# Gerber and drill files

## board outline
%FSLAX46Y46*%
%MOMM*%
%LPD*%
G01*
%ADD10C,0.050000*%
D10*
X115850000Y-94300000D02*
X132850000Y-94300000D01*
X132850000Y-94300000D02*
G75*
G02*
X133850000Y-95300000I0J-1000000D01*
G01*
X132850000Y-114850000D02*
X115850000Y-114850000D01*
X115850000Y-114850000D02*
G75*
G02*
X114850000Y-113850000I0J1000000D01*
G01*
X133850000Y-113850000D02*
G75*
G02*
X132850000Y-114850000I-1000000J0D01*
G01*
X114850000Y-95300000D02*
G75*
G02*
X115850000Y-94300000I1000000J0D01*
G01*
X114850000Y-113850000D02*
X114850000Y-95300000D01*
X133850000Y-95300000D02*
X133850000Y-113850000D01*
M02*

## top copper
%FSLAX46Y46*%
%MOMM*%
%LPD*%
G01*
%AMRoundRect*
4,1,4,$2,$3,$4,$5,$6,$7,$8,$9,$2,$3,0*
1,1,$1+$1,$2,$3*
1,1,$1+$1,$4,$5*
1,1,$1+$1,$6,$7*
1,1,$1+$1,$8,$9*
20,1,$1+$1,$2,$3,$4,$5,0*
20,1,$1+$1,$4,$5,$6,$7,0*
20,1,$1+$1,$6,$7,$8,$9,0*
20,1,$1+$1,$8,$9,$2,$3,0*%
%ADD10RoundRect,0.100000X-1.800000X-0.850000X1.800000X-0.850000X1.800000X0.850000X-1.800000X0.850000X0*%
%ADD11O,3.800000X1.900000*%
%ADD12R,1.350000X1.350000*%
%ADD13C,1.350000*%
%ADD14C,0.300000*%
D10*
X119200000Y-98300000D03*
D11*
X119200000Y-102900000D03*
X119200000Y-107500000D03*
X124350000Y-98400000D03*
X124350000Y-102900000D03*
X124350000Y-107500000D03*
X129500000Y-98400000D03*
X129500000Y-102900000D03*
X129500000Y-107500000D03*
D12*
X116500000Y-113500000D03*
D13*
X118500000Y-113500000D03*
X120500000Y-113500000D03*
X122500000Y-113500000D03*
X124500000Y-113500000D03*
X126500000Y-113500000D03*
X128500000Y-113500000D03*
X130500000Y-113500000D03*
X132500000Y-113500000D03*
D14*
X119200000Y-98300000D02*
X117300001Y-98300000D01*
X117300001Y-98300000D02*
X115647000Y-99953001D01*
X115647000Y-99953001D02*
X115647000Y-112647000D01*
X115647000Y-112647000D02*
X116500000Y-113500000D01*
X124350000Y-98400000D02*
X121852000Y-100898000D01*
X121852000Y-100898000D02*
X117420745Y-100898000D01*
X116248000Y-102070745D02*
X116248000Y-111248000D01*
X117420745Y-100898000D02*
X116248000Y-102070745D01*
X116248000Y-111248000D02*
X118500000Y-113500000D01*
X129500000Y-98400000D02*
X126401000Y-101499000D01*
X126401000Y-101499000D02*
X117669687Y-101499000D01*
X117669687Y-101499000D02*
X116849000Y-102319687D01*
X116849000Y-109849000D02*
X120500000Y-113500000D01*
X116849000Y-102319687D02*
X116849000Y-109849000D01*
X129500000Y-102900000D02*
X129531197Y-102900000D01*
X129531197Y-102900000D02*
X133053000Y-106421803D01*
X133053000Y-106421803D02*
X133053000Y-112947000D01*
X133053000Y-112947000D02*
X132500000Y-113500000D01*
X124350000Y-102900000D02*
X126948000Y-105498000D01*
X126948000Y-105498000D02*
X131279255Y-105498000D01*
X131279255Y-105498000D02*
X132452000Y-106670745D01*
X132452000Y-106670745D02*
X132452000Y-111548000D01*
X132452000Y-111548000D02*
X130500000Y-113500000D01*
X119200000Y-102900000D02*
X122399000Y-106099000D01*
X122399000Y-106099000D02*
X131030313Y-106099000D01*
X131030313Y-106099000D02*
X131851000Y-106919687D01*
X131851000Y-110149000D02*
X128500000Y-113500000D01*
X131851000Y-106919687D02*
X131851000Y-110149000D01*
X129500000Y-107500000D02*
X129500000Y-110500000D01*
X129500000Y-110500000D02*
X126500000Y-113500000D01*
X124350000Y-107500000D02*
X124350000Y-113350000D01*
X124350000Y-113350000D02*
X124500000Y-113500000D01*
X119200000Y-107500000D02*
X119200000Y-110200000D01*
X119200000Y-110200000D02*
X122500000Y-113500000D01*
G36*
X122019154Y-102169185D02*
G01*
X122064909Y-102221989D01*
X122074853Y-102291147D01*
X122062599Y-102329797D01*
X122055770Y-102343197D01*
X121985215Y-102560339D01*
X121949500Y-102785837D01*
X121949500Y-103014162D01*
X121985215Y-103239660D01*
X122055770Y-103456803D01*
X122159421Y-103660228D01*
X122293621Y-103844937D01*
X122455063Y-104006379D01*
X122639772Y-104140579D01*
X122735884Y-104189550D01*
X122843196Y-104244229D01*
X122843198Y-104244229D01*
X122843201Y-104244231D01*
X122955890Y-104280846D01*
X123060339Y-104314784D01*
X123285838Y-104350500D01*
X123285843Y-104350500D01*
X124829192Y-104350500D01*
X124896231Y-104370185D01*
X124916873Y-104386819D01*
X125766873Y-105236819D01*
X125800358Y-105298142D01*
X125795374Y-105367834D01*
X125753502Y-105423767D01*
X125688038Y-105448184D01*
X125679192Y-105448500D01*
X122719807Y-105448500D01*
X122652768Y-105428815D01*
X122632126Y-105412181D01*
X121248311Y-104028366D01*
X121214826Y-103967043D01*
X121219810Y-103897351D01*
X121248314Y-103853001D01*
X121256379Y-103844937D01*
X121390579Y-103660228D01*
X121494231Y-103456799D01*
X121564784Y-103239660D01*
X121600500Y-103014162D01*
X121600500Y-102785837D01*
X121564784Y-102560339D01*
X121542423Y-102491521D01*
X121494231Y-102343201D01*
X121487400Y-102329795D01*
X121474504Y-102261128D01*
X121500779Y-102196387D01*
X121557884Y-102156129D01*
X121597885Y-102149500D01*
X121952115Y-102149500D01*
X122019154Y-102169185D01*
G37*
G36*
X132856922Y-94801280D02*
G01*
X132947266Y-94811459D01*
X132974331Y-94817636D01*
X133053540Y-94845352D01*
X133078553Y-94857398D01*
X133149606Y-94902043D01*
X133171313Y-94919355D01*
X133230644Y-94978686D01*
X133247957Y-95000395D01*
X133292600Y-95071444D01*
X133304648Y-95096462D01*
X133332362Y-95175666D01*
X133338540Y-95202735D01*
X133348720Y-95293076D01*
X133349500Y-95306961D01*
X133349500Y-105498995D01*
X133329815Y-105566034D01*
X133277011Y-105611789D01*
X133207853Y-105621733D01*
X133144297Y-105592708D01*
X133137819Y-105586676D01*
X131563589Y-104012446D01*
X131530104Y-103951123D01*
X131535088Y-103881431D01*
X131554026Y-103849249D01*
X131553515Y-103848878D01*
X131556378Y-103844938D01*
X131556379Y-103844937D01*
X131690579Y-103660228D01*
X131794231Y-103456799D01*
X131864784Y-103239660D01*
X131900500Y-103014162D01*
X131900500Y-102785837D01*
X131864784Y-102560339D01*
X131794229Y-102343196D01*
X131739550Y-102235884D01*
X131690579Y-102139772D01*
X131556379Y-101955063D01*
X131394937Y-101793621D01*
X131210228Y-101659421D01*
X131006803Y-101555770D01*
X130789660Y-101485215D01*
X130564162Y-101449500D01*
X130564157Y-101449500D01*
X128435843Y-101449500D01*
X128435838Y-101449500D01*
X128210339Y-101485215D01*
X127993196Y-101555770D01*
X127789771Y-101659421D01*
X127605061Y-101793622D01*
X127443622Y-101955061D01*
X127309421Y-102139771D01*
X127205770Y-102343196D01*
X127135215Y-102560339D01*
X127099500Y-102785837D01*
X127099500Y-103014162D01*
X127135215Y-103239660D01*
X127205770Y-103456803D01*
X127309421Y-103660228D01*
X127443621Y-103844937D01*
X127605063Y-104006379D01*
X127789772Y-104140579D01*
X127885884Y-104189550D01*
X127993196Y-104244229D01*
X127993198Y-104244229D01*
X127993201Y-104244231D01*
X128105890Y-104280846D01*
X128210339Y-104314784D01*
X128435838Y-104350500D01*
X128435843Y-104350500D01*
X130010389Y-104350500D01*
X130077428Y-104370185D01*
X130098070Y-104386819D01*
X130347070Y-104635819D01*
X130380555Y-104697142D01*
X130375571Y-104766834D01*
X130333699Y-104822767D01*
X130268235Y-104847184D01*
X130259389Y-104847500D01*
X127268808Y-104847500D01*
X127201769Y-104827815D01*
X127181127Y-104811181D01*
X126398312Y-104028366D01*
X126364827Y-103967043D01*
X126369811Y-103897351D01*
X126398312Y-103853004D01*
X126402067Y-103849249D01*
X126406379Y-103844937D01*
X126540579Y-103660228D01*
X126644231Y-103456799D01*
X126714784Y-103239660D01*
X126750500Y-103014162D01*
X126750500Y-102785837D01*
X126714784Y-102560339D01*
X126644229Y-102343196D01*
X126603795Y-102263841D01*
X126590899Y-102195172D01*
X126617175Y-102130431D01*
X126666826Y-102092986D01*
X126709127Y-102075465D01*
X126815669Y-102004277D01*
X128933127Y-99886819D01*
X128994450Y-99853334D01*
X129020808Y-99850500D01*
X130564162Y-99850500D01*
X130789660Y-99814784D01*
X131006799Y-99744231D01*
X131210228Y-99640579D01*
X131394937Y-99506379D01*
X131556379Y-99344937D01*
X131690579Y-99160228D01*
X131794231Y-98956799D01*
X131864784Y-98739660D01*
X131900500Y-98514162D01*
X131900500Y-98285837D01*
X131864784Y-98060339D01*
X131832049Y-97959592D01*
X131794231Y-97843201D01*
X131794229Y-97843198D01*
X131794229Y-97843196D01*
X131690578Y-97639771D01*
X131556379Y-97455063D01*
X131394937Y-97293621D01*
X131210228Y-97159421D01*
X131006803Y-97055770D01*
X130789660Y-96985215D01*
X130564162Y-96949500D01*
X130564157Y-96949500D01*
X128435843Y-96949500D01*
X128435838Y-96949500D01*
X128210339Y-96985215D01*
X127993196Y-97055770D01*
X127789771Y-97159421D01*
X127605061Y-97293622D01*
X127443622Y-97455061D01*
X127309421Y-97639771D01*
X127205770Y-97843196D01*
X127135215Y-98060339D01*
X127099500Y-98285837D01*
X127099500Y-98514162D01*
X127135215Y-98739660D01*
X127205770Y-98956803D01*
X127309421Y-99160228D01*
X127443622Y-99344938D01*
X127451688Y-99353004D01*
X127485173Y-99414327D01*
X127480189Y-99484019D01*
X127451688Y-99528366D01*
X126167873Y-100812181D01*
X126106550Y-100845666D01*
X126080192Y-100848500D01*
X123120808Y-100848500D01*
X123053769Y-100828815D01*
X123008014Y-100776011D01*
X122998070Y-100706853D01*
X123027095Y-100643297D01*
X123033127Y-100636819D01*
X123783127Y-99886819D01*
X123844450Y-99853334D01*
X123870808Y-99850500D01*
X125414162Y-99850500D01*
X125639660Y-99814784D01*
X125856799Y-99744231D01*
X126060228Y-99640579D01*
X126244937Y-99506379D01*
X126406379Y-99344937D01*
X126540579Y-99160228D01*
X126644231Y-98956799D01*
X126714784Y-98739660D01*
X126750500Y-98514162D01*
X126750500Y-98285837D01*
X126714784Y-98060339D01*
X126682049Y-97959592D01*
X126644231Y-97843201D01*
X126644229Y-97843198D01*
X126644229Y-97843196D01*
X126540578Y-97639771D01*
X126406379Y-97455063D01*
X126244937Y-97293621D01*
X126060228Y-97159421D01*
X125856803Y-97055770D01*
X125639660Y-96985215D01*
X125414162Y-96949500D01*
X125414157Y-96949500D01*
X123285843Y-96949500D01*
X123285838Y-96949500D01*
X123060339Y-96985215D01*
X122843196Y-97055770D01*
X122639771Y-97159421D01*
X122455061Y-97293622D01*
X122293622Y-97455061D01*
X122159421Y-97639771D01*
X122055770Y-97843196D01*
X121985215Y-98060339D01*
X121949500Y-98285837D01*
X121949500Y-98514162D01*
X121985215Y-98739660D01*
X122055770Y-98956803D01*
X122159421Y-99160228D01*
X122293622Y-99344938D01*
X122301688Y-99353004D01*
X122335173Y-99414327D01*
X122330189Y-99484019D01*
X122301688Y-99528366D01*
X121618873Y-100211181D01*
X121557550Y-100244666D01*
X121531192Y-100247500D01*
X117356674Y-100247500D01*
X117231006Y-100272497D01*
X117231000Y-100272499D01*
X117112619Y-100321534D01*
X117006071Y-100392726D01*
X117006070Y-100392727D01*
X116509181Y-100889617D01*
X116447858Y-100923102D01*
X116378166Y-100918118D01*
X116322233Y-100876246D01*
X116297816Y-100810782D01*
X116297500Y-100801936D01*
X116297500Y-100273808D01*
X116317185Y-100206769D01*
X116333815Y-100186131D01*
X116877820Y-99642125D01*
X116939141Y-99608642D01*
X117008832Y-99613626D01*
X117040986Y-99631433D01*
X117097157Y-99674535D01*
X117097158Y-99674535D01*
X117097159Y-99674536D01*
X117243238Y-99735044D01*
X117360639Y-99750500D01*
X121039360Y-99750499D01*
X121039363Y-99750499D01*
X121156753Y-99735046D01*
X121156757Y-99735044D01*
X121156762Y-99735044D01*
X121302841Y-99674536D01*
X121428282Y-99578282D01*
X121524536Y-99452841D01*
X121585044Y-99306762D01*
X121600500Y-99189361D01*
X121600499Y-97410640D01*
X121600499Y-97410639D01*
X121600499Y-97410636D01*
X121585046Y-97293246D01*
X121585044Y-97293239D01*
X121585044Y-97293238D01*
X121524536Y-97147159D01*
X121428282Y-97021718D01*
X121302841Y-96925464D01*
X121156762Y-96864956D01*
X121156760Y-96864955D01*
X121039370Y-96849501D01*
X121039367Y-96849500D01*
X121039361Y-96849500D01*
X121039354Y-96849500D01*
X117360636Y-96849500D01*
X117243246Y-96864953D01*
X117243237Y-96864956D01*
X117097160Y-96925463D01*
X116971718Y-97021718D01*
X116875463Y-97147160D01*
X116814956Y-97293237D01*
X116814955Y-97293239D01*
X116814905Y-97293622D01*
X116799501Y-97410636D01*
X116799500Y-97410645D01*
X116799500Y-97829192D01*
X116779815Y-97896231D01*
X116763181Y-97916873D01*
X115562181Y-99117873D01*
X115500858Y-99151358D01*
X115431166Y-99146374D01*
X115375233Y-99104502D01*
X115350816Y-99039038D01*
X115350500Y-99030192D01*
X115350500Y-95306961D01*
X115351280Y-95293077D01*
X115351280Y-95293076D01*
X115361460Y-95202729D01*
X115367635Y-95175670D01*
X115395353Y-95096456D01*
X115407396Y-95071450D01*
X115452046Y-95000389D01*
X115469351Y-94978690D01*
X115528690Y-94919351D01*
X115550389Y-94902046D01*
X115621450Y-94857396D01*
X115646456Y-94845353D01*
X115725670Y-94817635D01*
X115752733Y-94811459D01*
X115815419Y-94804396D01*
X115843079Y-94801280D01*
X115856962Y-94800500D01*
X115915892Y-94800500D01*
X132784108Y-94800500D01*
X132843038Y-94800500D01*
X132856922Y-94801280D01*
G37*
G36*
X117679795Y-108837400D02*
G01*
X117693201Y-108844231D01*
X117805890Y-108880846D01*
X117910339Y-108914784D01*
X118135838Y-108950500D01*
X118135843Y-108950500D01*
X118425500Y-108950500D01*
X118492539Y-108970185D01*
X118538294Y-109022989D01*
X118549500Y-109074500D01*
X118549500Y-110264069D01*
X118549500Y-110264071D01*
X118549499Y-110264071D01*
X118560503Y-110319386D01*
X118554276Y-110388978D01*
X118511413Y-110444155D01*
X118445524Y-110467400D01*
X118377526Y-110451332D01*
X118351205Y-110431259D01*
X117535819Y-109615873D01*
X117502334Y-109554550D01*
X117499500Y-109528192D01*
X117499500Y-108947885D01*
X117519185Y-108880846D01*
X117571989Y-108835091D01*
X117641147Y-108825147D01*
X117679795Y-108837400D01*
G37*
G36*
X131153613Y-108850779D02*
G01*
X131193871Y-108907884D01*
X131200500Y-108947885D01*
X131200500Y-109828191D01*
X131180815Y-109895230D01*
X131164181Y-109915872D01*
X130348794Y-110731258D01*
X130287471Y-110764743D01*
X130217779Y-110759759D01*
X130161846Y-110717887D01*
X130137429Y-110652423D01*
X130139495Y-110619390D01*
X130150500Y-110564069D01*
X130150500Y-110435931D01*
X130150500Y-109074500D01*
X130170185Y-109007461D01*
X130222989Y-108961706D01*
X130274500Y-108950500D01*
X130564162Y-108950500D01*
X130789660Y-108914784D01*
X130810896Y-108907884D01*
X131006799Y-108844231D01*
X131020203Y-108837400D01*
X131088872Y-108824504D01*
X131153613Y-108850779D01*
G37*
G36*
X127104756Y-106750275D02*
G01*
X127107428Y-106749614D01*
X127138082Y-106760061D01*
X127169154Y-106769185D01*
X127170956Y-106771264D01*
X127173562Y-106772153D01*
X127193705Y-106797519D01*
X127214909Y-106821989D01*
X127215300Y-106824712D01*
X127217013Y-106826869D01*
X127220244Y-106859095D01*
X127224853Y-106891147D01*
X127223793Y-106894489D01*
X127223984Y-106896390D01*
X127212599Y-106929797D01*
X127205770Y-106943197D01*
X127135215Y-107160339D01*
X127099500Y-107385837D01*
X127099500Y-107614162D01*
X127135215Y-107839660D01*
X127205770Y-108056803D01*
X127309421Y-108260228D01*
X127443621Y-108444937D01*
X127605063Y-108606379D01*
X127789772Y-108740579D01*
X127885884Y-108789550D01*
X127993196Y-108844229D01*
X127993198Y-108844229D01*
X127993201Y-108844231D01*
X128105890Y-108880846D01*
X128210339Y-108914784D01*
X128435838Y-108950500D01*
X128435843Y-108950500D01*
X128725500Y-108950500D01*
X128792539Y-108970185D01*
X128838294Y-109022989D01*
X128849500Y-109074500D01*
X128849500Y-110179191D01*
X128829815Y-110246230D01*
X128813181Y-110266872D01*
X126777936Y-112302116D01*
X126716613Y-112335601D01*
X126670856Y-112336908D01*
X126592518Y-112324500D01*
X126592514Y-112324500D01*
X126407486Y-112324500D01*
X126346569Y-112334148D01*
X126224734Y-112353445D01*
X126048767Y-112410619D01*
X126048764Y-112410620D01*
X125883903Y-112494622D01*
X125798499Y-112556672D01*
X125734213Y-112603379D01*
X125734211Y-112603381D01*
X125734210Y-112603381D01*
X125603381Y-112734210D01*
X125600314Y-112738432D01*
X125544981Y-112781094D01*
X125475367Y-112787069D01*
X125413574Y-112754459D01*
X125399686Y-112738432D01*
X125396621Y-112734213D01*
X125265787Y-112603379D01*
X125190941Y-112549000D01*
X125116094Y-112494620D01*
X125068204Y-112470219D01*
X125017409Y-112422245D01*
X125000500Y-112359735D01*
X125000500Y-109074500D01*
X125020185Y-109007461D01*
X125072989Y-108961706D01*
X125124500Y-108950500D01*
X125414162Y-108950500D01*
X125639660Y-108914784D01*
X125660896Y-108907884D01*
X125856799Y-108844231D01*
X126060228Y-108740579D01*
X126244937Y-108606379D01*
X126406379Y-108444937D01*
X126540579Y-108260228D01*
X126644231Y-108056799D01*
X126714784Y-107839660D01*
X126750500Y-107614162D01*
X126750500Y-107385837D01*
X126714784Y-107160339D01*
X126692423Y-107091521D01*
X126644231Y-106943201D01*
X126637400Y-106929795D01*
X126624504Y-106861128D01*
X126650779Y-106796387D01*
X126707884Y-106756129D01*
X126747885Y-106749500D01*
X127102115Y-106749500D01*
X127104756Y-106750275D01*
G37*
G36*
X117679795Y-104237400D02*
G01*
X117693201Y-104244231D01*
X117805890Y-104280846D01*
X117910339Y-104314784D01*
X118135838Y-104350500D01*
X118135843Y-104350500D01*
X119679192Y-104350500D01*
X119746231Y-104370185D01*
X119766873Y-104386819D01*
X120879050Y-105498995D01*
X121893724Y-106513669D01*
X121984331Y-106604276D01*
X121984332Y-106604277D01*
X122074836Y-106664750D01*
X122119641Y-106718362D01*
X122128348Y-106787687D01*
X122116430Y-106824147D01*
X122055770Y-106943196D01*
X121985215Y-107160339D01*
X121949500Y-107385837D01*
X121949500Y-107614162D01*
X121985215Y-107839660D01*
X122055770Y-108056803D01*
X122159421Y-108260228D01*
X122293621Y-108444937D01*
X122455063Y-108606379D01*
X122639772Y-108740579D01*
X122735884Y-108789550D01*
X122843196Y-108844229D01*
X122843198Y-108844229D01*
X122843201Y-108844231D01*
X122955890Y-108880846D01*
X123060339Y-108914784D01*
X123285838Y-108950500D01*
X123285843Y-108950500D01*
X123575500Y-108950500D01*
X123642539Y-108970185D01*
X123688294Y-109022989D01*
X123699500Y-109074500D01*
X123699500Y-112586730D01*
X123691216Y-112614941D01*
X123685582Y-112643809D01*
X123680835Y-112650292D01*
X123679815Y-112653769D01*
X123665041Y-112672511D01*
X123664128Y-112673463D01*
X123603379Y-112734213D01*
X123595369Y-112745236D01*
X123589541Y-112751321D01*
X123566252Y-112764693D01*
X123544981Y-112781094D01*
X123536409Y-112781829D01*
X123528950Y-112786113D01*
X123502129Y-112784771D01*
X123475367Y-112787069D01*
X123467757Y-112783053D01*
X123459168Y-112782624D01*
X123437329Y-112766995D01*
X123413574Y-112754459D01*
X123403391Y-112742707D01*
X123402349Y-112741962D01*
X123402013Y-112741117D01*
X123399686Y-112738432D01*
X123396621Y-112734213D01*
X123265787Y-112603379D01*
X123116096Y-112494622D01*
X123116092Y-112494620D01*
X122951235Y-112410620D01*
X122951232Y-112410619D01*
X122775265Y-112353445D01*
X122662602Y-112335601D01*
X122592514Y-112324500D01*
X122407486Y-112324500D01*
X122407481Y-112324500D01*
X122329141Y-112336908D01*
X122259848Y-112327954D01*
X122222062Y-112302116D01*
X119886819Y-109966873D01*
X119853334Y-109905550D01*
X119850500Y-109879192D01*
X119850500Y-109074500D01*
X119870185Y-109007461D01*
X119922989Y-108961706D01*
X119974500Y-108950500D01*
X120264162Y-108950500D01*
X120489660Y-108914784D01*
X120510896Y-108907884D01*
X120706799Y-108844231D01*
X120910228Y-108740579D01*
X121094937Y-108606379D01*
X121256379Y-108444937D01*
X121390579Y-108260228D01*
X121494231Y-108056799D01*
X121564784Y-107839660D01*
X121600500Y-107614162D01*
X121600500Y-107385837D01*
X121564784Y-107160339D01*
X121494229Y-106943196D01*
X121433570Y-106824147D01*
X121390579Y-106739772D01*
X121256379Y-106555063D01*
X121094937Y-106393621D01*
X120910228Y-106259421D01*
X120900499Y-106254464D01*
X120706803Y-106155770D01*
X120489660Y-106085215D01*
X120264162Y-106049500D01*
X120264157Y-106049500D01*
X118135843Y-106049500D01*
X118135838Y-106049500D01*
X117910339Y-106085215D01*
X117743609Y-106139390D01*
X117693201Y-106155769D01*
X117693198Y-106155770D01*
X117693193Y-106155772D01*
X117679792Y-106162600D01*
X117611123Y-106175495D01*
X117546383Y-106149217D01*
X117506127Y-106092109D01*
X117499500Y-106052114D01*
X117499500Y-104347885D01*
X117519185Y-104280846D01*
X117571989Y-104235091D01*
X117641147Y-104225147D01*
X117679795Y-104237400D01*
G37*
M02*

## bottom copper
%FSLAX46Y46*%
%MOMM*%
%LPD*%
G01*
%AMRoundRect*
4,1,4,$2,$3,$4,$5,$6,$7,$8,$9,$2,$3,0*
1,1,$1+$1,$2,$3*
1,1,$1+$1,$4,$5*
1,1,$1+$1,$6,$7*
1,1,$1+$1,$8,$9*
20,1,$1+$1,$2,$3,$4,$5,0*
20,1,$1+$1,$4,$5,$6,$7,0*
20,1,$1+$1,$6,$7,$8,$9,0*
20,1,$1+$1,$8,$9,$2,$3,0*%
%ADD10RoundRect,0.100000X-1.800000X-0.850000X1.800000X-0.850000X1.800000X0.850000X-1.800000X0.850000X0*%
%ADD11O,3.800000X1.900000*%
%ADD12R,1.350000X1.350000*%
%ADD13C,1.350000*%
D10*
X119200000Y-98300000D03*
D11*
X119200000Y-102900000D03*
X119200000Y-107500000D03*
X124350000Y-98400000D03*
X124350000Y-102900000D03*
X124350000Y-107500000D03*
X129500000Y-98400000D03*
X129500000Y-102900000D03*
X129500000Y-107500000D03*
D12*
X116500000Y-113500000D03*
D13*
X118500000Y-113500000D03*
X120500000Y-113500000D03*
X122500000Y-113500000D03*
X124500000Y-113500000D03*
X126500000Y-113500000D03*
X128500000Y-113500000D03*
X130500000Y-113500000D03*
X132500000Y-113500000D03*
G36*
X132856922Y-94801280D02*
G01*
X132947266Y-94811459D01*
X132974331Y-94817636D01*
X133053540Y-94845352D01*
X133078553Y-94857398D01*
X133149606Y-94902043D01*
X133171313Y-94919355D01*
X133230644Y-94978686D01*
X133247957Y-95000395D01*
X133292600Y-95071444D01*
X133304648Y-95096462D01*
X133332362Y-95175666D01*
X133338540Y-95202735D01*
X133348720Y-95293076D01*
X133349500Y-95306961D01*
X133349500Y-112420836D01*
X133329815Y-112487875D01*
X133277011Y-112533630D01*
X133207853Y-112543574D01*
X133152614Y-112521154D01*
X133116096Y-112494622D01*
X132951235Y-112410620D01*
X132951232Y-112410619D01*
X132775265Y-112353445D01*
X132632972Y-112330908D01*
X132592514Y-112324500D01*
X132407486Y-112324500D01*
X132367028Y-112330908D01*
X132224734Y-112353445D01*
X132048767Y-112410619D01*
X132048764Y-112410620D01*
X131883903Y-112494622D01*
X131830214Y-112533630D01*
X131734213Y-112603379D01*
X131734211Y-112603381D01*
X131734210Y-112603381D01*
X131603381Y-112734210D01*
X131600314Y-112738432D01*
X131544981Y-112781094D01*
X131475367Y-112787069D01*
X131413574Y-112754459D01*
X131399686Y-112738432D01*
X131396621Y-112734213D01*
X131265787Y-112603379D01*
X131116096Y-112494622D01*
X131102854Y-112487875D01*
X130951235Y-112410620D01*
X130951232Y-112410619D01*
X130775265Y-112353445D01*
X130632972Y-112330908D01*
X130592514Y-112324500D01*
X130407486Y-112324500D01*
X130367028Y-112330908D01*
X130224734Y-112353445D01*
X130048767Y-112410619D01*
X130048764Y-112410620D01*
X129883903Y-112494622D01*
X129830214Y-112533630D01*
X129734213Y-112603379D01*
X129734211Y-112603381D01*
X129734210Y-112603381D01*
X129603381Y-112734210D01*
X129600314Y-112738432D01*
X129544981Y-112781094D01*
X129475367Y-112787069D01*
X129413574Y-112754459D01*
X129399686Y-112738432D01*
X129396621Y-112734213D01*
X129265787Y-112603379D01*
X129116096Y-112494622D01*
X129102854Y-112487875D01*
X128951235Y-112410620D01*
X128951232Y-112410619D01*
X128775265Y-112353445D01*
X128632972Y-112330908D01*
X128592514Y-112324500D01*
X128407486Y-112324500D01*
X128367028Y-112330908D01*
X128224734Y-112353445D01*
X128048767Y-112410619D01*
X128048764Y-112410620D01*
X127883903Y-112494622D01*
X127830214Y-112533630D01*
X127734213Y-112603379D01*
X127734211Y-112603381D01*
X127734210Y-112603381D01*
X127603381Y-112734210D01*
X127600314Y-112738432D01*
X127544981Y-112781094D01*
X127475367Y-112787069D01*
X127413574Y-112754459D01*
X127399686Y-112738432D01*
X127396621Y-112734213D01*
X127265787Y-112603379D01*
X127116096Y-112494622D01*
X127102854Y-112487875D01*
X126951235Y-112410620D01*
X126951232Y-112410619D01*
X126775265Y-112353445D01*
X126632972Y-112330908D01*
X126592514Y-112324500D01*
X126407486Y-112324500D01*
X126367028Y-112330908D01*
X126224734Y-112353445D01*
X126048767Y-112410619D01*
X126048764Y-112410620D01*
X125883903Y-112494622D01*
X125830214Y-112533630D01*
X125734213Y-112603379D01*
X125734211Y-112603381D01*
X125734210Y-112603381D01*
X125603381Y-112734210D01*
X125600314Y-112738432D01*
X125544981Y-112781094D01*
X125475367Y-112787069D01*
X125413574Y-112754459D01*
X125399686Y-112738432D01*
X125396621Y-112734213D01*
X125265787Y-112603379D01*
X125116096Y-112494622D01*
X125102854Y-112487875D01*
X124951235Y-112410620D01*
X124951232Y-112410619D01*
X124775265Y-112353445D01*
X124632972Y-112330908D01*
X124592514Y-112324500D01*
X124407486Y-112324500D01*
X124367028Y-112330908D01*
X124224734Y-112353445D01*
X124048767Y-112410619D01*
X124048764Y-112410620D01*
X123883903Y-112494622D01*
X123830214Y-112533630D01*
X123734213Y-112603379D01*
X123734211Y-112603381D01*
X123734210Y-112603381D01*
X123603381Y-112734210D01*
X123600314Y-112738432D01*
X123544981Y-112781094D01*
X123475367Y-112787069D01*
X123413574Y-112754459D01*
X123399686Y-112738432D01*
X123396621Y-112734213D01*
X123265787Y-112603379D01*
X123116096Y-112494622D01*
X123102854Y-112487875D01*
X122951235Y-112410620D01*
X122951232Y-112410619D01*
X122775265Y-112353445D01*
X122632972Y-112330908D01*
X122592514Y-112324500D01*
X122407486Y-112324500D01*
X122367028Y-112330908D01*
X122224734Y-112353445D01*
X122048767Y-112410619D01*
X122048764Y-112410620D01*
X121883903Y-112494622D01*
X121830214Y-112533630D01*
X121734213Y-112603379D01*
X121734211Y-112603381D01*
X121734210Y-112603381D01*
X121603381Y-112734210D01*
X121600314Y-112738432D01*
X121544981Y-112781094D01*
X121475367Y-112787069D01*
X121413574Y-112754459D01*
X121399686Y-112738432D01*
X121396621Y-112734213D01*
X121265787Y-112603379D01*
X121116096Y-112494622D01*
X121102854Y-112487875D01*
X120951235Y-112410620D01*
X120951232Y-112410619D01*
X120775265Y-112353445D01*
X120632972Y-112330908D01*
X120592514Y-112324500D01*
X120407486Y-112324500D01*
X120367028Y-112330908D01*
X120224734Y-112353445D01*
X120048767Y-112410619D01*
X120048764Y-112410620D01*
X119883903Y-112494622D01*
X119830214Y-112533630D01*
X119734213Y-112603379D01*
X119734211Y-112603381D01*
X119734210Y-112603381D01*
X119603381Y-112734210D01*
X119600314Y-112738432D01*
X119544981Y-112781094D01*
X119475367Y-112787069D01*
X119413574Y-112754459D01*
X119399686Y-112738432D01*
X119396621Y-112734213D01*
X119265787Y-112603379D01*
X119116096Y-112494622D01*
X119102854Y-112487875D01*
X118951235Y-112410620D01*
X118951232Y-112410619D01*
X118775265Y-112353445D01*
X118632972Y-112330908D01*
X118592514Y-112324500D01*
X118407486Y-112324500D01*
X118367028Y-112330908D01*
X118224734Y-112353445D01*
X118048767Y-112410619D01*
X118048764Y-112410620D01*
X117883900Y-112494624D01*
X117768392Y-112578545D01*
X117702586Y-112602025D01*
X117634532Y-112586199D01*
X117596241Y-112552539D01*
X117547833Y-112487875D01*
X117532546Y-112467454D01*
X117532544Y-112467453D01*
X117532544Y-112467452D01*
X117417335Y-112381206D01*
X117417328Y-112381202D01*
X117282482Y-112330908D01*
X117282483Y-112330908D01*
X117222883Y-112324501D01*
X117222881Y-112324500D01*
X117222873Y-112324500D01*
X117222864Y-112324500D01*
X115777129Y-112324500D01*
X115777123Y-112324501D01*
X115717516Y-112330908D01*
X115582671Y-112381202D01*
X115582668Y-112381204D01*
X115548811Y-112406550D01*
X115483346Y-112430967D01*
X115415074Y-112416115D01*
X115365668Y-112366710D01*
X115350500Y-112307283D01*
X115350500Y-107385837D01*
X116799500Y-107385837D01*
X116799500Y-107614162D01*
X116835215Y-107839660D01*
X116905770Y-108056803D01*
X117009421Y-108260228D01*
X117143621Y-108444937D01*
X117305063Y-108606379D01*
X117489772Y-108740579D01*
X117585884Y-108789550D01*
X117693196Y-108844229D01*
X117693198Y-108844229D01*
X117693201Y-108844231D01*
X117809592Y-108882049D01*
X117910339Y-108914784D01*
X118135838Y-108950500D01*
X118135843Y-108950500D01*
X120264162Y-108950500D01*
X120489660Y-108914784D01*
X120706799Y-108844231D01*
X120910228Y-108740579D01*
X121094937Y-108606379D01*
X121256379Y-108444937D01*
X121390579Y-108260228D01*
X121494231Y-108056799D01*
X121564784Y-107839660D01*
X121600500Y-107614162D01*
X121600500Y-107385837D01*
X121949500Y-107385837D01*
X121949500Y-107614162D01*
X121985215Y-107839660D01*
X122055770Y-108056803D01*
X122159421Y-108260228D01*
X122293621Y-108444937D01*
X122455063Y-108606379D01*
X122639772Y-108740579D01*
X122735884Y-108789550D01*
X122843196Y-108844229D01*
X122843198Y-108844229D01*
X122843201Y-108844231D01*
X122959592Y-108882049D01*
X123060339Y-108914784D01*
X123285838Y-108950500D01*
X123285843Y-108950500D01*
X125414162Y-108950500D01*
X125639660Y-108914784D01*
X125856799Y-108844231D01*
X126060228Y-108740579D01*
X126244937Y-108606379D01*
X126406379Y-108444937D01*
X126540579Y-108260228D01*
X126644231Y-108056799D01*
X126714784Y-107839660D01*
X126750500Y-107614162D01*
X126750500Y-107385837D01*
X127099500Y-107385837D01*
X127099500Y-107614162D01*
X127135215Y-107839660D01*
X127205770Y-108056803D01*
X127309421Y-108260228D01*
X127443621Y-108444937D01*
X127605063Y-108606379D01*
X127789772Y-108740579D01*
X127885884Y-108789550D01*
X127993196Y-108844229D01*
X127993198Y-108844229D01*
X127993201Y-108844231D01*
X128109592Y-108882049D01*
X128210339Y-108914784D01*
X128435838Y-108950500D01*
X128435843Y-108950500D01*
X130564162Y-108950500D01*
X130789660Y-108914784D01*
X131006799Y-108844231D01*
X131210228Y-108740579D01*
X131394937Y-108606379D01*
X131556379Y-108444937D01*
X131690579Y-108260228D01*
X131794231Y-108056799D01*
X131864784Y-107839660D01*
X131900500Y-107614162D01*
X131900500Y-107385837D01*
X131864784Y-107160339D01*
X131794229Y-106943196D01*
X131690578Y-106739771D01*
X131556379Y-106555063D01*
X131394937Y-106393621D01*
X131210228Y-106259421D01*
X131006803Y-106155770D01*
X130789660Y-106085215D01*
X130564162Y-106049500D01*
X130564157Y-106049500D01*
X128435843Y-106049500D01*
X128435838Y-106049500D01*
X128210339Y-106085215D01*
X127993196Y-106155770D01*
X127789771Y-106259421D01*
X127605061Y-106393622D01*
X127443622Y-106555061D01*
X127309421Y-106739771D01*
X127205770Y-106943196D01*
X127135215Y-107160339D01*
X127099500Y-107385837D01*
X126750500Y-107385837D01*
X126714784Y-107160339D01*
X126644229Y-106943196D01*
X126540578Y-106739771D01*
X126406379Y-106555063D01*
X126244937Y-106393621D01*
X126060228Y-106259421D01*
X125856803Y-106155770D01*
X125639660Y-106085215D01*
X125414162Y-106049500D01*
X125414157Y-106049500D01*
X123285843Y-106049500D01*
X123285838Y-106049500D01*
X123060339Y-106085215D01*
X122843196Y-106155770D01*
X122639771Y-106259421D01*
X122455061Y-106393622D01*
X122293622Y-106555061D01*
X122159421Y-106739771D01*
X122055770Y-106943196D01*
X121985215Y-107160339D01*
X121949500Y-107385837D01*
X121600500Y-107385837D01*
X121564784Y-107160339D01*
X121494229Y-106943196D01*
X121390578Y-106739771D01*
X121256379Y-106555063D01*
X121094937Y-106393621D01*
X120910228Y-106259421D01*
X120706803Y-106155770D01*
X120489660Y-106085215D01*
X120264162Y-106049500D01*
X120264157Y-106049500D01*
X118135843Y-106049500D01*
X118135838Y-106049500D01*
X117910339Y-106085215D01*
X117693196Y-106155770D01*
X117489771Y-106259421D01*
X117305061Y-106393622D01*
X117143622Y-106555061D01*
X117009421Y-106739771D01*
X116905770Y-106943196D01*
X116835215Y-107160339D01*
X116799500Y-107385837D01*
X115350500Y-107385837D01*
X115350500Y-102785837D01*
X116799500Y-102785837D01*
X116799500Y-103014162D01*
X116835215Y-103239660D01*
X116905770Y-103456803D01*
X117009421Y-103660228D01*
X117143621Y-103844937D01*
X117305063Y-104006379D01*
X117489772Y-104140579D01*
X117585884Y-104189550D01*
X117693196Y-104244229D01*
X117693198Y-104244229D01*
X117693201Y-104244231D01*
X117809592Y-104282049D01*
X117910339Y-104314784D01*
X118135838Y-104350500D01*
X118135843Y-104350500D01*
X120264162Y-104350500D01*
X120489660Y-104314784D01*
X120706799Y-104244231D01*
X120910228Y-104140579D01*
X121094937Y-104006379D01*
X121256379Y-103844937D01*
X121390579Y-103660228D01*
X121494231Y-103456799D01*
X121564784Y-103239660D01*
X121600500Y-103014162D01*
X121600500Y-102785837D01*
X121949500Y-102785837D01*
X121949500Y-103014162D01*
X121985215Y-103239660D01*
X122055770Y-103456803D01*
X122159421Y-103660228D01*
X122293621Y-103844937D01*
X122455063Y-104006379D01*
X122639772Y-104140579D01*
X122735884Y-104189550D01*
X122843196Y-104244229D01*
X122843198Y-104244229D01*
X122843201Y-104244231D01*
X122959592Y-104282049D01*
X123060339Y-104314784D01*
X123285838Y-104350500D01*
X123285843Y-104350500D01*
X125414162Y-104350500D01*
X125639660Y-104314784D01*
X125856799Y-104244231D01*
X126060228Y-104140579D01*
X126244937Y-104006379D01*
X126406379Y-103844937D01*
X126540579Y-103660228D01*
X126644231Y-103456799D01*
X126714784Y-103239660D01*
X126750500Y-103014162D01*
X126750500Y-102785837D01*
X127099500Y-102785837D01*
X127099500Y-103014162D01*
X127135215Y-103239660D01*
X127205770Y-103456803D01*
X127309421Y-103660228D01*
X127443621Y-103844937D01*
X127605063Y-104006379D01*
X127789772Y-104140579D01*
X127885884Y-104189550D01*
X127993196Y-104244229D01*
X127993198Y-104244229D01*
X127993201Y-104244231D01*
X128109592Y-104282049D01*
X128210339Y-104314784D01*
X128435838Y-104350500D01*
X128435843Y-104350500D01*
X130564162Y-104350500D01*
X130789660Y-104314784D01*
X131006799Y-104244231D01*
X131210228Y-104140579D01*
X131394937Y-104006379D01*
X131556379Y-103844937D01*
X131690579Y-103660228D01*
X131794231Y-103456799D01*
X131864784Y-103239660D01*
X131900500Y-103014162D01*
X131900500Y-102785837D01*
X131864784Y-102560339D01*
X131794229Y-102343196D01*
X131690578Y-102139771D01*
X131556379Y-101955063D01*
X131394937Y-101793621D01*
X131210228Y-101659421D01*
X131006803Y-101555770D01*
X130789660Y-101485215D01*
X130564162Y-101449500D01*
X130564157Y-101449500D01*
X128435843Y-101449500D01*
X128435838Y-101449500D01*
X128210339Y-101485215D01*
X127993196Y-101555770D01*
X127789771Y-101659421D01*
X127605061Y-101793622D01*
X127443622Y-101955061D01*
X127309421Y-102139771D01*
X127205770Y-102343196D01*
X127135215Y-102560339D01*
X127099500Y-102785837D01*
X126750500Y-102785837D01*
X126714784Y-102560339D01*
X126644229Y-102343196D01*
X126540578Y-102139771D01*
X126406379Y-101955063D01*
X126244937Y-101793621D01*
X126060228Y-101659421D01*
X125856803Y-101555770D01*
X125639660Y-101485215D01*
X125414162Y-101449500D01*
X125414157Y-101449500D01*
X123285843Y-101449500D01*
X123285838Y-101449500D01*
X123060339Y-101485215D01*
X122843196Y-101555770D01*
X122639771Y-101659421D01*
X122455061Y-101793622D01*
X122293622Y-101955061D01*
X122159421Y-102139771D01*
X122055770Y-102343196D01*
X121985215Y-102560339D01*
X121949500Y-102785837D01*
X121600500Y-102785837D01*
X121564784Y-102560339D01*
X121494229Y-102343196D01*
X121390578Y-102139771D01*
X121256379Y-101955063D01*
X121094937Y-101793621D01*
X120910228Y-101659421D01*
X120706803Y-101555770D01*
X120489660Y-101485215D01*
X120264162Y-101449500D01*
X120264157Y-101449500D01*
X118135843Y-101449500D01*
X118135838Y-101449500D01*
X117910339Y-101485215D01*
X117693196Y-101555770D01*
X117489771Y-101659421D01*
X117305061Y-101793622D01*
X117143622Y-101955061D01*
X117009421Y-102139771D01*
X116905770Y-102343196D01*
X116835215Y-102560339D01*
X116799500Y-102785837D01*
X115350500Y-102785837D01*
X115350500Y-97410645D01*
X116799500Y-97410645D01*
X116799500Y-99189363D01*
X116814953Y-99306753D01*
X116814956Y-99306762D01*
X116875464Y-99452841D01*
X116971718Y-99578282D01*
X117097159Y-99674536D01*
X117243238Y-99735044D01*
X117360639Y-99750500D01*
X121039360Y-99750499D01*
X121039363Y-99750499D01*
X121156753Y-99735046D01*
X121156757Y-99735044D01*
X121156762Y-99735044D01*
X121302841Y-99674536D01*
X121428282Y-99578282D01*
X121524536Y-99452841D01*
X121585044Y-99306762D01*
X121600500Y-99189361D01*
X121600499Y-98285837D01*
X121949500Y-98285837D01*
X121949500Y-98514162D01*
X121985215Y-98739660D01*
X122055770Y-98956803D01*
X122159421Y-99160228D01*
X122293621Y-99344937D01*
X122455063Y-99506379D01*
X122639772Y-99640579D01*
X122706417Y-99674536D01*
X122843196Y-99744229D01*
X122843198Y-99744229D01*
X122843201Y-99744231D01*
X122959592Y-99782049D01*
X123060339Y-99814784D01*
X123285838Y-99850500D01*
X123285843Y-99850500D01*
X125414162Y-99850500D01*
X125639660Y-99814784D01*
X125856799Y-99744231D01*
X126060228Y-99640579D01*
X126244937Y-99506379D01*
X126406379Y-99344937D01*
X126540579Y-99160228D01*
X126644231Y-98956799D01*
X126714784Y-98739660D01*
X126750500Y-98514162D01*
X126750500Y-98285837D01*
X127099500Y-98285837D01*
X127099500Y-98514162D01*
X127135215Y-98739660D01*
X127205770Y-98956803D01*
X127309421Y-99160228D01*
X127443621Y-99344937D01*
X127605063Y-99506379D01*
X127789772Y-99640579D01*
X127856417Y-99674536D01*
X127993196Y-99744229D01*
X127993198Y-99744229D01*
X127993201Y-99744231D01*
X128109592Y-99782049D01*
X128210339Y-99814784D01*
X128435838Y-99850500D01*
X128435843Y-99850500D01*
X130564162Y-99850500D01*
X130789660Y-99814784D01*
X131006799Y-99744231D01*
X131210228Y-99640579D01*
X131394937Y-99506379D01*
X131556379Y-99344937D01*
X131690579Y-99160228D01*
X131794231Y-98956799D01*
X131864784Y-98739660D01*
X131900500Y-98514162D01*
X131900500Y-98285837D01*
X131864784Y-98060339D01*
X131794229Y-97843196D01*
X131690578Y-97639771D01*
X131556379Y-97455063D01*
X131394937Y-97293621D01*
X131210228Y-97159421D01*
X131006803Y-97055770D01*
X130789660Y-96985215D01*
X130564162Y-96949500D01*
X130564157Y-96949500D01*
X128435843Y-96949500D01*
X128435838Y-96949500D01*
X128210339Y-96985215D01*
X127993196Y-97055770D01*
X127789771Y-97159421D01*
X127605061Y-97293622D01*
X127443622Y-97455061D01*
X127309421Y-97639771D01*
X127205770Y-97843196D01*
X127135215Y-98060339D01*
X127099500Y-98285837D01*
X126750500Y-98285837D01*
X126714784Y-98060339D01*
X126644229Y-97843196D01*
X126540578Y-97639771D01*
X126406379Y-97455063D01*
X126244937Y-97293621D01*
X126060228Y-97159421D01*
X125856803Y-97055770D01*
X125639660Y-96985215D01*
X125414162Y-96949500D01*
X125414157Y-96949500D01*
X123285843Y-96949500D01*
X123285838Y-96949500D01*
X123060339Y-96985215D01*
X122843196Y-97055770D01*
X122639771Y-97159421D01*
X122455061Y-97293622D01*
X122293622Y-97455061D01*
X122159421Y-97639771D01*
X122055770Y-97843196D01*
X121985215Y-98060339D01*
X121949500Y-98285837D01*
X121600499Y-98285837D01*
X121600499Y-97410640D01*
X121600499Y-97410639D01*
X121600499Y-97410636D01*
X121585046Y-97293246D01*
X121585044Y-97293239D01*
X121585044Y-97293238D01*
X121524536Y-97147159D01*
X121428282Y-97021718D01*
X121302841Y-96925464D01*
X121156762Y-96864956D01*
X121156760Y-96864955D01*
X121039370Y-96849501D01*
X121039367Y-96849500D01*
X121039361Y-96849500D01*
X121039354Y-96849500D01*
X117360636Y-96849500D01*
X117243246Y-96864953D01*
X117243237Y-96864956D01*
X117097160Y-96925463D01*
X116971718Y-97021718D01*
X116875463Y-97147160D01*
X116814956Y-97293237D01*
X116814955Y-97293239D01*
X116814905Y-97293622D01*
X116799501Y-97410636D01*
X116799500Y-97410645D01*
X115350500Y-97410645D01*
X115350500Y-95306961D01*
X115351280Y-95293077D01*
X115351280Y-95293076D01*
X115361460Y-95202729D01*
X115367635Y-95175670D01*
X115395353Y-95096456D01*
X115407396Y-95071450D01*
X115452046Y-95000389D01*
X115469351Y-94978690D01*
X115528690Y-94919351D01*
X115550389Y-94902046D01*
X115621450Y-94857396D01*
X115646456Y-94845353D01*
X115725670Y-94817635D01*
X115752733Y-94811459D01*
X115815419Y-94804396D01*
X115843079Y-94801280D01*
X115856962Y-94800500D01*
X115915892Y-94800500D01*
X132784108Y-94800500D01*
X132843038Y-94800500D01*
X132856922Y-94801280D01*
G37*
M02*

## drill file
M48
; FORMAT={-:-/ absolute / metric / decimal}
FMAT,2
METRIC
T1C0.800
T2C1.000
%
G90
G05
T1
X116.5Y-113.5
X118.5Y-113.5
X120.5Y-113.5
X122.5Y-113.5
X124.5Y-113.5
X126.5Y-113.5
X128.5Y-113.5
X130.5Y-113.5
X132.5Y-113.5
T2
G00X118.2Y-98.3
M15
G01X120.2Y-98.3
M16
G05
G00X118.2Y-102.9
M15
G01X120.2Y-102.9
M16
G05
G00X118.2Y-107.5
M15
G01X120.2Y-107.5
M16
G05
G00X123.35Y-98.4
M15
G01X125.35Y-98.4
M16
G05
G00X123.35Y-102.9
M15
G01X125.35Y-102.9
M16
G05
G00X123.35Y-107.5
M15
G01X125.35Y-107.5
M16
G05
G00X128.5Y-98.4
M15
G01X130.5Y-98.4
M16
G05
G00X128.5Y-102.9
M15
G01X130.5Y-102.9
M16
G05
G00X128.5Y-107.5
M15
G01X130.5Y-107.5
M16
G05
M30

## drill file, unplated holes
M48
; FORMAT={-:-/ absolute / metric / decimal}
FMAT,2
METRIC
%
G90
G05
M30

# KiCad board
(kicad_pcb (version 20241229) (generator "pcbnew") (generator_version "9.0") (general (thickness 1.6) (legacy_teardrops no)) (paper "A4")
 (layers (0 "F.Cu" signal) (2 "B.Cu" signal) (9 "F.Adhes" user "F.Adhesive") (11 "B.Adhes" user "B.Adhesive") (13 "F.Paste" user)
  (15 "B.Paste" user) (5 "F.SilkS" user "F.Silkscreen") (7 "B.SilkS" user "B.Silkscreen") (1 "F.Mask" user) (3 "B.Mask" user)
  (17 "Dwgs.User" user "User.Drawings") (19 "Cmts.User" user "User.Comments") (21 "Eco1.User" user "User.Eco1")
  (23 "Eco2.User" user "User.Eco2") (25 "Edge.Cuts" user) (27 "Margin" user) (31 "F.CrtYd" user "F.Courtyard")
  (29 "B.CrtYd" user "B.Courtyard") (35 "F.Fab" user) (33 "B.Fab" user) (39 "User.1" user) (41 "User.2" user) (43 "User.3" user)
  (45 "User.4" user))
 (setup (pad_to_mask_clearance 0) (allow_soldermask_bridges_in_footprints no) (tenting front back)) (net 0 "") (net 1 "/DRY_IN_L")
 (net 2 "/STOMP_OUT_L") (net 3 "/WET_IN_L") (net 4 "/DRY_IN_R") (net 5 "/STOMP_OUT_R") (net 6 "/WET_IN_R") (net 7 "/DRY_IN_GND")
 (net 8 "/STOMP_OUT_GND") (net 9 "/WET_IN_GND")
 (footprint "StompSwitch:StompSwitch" (layer "F.Cu") (at 119.2 98.3)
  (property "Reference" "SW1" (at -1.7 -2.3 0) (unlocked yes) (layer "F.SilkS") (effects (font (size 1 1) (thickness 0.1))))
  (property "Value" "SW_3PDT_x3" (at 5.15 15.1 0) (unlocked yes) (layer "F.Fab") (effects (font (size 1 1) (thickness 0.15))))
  (pad "1" thru_hole roundrect (at 0 0) (size 3.8 1.9) (drill oval 3 1) (layers "*.Cu" "*.Mask") (remove_unused_layers no)
   (roundrect_rratio 0.05263157895) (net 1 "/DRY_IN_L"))
  (pad "2" thru_hole oval (at 0 4.6) (size 3.8 1.9) (drill oval 3 1) (layers "*.Cu" "*.Mask") (remove_unused_layers no)
   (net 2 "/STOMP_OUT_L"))
  (pad "3" thru_hole oval (at 0 9.2) (size 3.8 1.9) (drill oval 3 1) (layers "*.Cu" "*.Mask") (remove_unused_layers no) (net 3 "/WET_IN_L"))
  (pad "4" thru_hole oval (at 5.15 0.1) (size 3.8 1.9) (drill oval 3 1) (layers "*.Cu" "*.Mask") (remove_unused_layers no)
   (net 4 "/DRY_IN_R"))
  (pad "5" thru_hole oval (at 5.15 4.6) (size 3.8 1.9) (drill oval 3 1) (layers "*.Cu" "*.Mask") (remove_unused_layers no)
   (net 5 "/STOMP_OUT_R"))
  (pad "6" thru_hole oval (at 5.15 9.2) (size 3.8 1.9) (drill oval 3 1) (layers "*.Cu" "*.Mask") (remove_unused_layers no)
   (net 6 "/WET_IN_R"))
  (pad "7" thru_hole oval (at 10.3 0.1) (size 3.8 1.9) (drill oval 3 1) (layers "*.Cu" "*.Mask") (remove_unused_layers no)
   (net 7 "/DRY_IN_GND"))
  (pad "8" thru_hole oval (at 10.3 4.6) (size 3.8 1.9) (drill oval 3 1) (layers "*.Cu" "*.Mask") (remove_unused_layers no)
   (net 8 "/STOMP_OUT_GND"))
  (pad "9" thru_hole oval (at 10.3 9.2) (size 3.8 1.9) (drill oval 3 1) (layers "*.Cu" "*.Mask") (remove_unused_layers no)
   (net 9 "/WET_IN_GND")))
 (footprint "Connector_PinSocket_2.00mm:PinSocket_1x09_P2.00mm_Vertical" (layer "F.Cu") (at 116.5 113.5 90)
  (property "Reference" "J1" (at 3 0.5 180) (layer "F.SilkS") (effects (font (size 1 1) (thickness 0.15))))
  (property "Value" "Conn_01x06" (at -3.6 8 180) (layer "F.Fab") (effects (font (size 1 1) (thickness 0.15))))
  (pad "1" thru_hole rect (at 0 0 90) (size 1.35 1.35) (drill 0.8) (layers "*.Cu" "*.Mask") (remove_unused_layers no) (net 1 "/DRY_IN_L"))
  (pad "2" thru_hole circle (at 0 2 90) (size 1.35 1.35) (drill 0.8) (layers "*.Cu" "*.Mask") (remove_unused_layers no) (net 4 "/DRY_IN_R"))
  (pad "3" thru_hole circle (at 0 4 90) (size 1.35 1.35) (drill 0.8) (layers "*.Cu" "*.Mask") (remove_unused_layers no)
   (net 7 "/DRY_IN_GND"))
  (pad "4" thru_hole circle (at 0 6 90) (size 1.35 1.35) (drill 0.8) (layers "*.Cu" "*.Mask") (remove_unused_layers no) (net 3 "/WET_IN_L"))
  (pad "5" thru_hole circle (at 0 8 90) (size 1.35 1.35) (drill 0.8) (layers "*.Cu" "*.Mask") (remove_unused_layers no) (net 6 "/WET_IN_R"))
  (pad "6" thru_hole circle (at 0 10 90) (size 1.35 1.35) (drill 0.8) (layers "*.Cu" "*.Mask") (remove_unused_layers no)
   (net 9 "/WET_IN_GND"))
  (pad "7" thru_hole circle (at 0 12 90) (size 1.35 1.35) (drill 0.8) (layers "*.Cu" "*.Mask") (remove_unused_layers no)
   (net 2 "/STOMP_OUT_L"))
  (pad "8" thru_hole circle (at 0 14 90) (size 1.35 1.35) (drill 0.8) (layers "*.Cu" "*.Mask") (remove_unused_layers no)
   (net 5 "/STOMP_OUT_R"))
  (pad "9" thru_hole circle (at 0 16 90) (size 1.35 1.35) (drill 0.8) (layers "*.Cu" "*.Mask") (remove_unused_layers no)
   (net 8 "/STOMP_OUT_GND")))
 (gr_line (start 115.85 94.3) (end 132.85 94.3) (stroke (width 0.05) (type default)) (layer "Edge.Cuts"))
 (gr_arc (start 132.85 94.3) (mid 133.557107 94.592893) (end 133.85 95.3) (stroke (width 0.05) (type default)) (layer "Edge.Cuts"))
 (gr_line (start 132.85 114.85) (end 115.85 114.85) (stroke (width 0.05) (type default)) (layer "Edge.Cuts"))
 (gr_arc (start 115.85 114.85) (mid 115.142893 114.557107) (end 114.85 113.85) (stroke (width 0.05) (type default)) (layer "Edge.Cuts"))
 (gr_arc (start 133.85 113.85) (mid 133.557107 114.557107) (end 132.85 114.85) (stroke (width 0.05) (type default)) (layer "Edge.Cuts"))
 (gr_arc (start 114.85 95.3) (mid 115.142893 94.592893) (end 115.85 94.3) (stroke (width 0.05) (type default)) (layer "Edge.Cuts"))
 (gr_line (start 114.85 113.85) (end 114.85 95.3) (stroke (width 0.05) (type default)) (layer "Edge.Cuts"))
 (gr_line (start 133.85 95.3) (end 133.85 113.85) (stroke (width 0.05) (type default)) (layer "Edge.Cuts"))
 (segment (start 116.248 111.248) (end 118.5 113.5) (width 0.3) (layer "F.Cu") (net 4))
 (segment (start 124.35 98.4) (end 121.852 100.898) (width 0.3) (layer "F.Cu") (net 4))
 (segment (start 116.248 102.070745) (end 116.248 111.248) (width 0.3) (layer "F.Cu") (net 4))
 (segment (start 121.852 100.898) (end 117.420745 100.898) (width 0.3) (layer "F.Cu") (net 4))
 (segment (start 117.420745 100.898) (end 116.248 102.070745) (width 0.3) (layer "F.Cu") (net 4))
 (segment (start 124.35 107.5) (end 124.35 113.35) (width 0.3) (layer "F.Cu") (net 6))
 (segment (start 124.35 113.35) (end 124.5 113.5) (width 0.3) (layer "F.Cu") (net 6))
 (segment (start 117.300001 98.3) (end 115.647 99.953001) (width 0.3) (layer "F.Cu") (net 1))
 (segment (start 115.647 112.647) (end 116.5 113.5) (width 0.3) (layer "F.Cu") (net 1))
 (segment (start 119.2 98.3) (end 117.300001 98.3) (width 0.3) (layer "F.Cu") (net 1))
 (segment (start 115.647 99.953001) (end 115.647 112.647) (width 0.3) (layer "F.Cu") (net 1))
 (segment (start 131.851 110.149) (end 128.5 113.5) (width 0.3) (layer "F.Cu") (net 2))
 (segment (start 122.399 106.099) (end 131.030313 106.099) (width 0.3) (layer "F.Cu") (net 2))
 (segment (start 119.2 102.9) (end 122.399 106.099) (width 0.3) (layer "F.Cu") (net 2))
 (segment (start 131.851 106.919687) (end 131.851 110.149) (width 0.3) (layer "F.Cu") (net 2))
 (segment (start 131.030313 106.099) (end 131.851 106.919687) (width 0.3) (layer "F.Cu") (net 2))
 (segment (start 129.5 102.9) (end 129.531197 102.9) (width 0.3) (layer "F.Cu") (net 8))
 (segment (start 133.053 106.421803) (end 133.053 112.947) (width 0.3) (layer "F.Cu") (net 8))
 (segment (start 129.531197 102.9) (end 133.053 106.421803) (width 0.3) (layer "F.Cu") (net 8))
 (segment (start 133.053 112.947) (end 132.5 113.5) (width 0.3) (layer "F.Cu") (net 8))
 (segment (start 126.948 105.498) (end 131.279255 105.498) (width 0.3) (layer "F.Cu") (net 5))
 (segment (start 131.279255 105.498) (end 132.452 106.670745) (width 0.3) (layer "F.Cu") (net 5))
 (segment (start 132.452 111.548) (end 130.5 113.5) (width 0.3) (layer "F.Cu") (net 5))
 (segment (start 132.452 106.670745) (end 132.452 111.548) (width 0.3) (layer "F.Cu") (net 5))
 (segment (start 124.35 102.9) (end 126.948 105.498) (width 0.3) (layer "F.Cu") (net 5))
 (segment (start 129.5 107.5) (end 129.5 110.5) (width 0.3) (layer "F.Cu") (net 9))
 (segment (start 129.5 110.5) (end 126.5 113.5) (width 0.3) (layer "F.Cu") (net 9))
 (segment (start 129.5 98.4) (end 126.401 101.499) (width 0.3) (layer "F.Cu") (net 7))
 (segment (start 126.401 101.499) (end 117.669687 101.499) (width 0.3) (layer "F.Cu") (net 7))
 (segment (start 117.669687 101.499) (end 116.849 102.319687) (width 0.3) (layer "F.Cu") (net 7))
 (segment (start 116.849 109.849) (end 120.5 113.5) (width 0.3) (layer "F.Cu") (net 7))
 (segment (start 116.849 102.319687) (end 116.849 109.849) (width 0.3) (layer "F.Cu") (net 7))
 (segment (start 119.2 110.2) (end 122.5 113.5) (width 0.3) (layer "F.Cu") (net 3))
 (segment (start 119.2 107.5) (end 119.2 110.2) (width 0.3) (layer "F.Cu") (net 3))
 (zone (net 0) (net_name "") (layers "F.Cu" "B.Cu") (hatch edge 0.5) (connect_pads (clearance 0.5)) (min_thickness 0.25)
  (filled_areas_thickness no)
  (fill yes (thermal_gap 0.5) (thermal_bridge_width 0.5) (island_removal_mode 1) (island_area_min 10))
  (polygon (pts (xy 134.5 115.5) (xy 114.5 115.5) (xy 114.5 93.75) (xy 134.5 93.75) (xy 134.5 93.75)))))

